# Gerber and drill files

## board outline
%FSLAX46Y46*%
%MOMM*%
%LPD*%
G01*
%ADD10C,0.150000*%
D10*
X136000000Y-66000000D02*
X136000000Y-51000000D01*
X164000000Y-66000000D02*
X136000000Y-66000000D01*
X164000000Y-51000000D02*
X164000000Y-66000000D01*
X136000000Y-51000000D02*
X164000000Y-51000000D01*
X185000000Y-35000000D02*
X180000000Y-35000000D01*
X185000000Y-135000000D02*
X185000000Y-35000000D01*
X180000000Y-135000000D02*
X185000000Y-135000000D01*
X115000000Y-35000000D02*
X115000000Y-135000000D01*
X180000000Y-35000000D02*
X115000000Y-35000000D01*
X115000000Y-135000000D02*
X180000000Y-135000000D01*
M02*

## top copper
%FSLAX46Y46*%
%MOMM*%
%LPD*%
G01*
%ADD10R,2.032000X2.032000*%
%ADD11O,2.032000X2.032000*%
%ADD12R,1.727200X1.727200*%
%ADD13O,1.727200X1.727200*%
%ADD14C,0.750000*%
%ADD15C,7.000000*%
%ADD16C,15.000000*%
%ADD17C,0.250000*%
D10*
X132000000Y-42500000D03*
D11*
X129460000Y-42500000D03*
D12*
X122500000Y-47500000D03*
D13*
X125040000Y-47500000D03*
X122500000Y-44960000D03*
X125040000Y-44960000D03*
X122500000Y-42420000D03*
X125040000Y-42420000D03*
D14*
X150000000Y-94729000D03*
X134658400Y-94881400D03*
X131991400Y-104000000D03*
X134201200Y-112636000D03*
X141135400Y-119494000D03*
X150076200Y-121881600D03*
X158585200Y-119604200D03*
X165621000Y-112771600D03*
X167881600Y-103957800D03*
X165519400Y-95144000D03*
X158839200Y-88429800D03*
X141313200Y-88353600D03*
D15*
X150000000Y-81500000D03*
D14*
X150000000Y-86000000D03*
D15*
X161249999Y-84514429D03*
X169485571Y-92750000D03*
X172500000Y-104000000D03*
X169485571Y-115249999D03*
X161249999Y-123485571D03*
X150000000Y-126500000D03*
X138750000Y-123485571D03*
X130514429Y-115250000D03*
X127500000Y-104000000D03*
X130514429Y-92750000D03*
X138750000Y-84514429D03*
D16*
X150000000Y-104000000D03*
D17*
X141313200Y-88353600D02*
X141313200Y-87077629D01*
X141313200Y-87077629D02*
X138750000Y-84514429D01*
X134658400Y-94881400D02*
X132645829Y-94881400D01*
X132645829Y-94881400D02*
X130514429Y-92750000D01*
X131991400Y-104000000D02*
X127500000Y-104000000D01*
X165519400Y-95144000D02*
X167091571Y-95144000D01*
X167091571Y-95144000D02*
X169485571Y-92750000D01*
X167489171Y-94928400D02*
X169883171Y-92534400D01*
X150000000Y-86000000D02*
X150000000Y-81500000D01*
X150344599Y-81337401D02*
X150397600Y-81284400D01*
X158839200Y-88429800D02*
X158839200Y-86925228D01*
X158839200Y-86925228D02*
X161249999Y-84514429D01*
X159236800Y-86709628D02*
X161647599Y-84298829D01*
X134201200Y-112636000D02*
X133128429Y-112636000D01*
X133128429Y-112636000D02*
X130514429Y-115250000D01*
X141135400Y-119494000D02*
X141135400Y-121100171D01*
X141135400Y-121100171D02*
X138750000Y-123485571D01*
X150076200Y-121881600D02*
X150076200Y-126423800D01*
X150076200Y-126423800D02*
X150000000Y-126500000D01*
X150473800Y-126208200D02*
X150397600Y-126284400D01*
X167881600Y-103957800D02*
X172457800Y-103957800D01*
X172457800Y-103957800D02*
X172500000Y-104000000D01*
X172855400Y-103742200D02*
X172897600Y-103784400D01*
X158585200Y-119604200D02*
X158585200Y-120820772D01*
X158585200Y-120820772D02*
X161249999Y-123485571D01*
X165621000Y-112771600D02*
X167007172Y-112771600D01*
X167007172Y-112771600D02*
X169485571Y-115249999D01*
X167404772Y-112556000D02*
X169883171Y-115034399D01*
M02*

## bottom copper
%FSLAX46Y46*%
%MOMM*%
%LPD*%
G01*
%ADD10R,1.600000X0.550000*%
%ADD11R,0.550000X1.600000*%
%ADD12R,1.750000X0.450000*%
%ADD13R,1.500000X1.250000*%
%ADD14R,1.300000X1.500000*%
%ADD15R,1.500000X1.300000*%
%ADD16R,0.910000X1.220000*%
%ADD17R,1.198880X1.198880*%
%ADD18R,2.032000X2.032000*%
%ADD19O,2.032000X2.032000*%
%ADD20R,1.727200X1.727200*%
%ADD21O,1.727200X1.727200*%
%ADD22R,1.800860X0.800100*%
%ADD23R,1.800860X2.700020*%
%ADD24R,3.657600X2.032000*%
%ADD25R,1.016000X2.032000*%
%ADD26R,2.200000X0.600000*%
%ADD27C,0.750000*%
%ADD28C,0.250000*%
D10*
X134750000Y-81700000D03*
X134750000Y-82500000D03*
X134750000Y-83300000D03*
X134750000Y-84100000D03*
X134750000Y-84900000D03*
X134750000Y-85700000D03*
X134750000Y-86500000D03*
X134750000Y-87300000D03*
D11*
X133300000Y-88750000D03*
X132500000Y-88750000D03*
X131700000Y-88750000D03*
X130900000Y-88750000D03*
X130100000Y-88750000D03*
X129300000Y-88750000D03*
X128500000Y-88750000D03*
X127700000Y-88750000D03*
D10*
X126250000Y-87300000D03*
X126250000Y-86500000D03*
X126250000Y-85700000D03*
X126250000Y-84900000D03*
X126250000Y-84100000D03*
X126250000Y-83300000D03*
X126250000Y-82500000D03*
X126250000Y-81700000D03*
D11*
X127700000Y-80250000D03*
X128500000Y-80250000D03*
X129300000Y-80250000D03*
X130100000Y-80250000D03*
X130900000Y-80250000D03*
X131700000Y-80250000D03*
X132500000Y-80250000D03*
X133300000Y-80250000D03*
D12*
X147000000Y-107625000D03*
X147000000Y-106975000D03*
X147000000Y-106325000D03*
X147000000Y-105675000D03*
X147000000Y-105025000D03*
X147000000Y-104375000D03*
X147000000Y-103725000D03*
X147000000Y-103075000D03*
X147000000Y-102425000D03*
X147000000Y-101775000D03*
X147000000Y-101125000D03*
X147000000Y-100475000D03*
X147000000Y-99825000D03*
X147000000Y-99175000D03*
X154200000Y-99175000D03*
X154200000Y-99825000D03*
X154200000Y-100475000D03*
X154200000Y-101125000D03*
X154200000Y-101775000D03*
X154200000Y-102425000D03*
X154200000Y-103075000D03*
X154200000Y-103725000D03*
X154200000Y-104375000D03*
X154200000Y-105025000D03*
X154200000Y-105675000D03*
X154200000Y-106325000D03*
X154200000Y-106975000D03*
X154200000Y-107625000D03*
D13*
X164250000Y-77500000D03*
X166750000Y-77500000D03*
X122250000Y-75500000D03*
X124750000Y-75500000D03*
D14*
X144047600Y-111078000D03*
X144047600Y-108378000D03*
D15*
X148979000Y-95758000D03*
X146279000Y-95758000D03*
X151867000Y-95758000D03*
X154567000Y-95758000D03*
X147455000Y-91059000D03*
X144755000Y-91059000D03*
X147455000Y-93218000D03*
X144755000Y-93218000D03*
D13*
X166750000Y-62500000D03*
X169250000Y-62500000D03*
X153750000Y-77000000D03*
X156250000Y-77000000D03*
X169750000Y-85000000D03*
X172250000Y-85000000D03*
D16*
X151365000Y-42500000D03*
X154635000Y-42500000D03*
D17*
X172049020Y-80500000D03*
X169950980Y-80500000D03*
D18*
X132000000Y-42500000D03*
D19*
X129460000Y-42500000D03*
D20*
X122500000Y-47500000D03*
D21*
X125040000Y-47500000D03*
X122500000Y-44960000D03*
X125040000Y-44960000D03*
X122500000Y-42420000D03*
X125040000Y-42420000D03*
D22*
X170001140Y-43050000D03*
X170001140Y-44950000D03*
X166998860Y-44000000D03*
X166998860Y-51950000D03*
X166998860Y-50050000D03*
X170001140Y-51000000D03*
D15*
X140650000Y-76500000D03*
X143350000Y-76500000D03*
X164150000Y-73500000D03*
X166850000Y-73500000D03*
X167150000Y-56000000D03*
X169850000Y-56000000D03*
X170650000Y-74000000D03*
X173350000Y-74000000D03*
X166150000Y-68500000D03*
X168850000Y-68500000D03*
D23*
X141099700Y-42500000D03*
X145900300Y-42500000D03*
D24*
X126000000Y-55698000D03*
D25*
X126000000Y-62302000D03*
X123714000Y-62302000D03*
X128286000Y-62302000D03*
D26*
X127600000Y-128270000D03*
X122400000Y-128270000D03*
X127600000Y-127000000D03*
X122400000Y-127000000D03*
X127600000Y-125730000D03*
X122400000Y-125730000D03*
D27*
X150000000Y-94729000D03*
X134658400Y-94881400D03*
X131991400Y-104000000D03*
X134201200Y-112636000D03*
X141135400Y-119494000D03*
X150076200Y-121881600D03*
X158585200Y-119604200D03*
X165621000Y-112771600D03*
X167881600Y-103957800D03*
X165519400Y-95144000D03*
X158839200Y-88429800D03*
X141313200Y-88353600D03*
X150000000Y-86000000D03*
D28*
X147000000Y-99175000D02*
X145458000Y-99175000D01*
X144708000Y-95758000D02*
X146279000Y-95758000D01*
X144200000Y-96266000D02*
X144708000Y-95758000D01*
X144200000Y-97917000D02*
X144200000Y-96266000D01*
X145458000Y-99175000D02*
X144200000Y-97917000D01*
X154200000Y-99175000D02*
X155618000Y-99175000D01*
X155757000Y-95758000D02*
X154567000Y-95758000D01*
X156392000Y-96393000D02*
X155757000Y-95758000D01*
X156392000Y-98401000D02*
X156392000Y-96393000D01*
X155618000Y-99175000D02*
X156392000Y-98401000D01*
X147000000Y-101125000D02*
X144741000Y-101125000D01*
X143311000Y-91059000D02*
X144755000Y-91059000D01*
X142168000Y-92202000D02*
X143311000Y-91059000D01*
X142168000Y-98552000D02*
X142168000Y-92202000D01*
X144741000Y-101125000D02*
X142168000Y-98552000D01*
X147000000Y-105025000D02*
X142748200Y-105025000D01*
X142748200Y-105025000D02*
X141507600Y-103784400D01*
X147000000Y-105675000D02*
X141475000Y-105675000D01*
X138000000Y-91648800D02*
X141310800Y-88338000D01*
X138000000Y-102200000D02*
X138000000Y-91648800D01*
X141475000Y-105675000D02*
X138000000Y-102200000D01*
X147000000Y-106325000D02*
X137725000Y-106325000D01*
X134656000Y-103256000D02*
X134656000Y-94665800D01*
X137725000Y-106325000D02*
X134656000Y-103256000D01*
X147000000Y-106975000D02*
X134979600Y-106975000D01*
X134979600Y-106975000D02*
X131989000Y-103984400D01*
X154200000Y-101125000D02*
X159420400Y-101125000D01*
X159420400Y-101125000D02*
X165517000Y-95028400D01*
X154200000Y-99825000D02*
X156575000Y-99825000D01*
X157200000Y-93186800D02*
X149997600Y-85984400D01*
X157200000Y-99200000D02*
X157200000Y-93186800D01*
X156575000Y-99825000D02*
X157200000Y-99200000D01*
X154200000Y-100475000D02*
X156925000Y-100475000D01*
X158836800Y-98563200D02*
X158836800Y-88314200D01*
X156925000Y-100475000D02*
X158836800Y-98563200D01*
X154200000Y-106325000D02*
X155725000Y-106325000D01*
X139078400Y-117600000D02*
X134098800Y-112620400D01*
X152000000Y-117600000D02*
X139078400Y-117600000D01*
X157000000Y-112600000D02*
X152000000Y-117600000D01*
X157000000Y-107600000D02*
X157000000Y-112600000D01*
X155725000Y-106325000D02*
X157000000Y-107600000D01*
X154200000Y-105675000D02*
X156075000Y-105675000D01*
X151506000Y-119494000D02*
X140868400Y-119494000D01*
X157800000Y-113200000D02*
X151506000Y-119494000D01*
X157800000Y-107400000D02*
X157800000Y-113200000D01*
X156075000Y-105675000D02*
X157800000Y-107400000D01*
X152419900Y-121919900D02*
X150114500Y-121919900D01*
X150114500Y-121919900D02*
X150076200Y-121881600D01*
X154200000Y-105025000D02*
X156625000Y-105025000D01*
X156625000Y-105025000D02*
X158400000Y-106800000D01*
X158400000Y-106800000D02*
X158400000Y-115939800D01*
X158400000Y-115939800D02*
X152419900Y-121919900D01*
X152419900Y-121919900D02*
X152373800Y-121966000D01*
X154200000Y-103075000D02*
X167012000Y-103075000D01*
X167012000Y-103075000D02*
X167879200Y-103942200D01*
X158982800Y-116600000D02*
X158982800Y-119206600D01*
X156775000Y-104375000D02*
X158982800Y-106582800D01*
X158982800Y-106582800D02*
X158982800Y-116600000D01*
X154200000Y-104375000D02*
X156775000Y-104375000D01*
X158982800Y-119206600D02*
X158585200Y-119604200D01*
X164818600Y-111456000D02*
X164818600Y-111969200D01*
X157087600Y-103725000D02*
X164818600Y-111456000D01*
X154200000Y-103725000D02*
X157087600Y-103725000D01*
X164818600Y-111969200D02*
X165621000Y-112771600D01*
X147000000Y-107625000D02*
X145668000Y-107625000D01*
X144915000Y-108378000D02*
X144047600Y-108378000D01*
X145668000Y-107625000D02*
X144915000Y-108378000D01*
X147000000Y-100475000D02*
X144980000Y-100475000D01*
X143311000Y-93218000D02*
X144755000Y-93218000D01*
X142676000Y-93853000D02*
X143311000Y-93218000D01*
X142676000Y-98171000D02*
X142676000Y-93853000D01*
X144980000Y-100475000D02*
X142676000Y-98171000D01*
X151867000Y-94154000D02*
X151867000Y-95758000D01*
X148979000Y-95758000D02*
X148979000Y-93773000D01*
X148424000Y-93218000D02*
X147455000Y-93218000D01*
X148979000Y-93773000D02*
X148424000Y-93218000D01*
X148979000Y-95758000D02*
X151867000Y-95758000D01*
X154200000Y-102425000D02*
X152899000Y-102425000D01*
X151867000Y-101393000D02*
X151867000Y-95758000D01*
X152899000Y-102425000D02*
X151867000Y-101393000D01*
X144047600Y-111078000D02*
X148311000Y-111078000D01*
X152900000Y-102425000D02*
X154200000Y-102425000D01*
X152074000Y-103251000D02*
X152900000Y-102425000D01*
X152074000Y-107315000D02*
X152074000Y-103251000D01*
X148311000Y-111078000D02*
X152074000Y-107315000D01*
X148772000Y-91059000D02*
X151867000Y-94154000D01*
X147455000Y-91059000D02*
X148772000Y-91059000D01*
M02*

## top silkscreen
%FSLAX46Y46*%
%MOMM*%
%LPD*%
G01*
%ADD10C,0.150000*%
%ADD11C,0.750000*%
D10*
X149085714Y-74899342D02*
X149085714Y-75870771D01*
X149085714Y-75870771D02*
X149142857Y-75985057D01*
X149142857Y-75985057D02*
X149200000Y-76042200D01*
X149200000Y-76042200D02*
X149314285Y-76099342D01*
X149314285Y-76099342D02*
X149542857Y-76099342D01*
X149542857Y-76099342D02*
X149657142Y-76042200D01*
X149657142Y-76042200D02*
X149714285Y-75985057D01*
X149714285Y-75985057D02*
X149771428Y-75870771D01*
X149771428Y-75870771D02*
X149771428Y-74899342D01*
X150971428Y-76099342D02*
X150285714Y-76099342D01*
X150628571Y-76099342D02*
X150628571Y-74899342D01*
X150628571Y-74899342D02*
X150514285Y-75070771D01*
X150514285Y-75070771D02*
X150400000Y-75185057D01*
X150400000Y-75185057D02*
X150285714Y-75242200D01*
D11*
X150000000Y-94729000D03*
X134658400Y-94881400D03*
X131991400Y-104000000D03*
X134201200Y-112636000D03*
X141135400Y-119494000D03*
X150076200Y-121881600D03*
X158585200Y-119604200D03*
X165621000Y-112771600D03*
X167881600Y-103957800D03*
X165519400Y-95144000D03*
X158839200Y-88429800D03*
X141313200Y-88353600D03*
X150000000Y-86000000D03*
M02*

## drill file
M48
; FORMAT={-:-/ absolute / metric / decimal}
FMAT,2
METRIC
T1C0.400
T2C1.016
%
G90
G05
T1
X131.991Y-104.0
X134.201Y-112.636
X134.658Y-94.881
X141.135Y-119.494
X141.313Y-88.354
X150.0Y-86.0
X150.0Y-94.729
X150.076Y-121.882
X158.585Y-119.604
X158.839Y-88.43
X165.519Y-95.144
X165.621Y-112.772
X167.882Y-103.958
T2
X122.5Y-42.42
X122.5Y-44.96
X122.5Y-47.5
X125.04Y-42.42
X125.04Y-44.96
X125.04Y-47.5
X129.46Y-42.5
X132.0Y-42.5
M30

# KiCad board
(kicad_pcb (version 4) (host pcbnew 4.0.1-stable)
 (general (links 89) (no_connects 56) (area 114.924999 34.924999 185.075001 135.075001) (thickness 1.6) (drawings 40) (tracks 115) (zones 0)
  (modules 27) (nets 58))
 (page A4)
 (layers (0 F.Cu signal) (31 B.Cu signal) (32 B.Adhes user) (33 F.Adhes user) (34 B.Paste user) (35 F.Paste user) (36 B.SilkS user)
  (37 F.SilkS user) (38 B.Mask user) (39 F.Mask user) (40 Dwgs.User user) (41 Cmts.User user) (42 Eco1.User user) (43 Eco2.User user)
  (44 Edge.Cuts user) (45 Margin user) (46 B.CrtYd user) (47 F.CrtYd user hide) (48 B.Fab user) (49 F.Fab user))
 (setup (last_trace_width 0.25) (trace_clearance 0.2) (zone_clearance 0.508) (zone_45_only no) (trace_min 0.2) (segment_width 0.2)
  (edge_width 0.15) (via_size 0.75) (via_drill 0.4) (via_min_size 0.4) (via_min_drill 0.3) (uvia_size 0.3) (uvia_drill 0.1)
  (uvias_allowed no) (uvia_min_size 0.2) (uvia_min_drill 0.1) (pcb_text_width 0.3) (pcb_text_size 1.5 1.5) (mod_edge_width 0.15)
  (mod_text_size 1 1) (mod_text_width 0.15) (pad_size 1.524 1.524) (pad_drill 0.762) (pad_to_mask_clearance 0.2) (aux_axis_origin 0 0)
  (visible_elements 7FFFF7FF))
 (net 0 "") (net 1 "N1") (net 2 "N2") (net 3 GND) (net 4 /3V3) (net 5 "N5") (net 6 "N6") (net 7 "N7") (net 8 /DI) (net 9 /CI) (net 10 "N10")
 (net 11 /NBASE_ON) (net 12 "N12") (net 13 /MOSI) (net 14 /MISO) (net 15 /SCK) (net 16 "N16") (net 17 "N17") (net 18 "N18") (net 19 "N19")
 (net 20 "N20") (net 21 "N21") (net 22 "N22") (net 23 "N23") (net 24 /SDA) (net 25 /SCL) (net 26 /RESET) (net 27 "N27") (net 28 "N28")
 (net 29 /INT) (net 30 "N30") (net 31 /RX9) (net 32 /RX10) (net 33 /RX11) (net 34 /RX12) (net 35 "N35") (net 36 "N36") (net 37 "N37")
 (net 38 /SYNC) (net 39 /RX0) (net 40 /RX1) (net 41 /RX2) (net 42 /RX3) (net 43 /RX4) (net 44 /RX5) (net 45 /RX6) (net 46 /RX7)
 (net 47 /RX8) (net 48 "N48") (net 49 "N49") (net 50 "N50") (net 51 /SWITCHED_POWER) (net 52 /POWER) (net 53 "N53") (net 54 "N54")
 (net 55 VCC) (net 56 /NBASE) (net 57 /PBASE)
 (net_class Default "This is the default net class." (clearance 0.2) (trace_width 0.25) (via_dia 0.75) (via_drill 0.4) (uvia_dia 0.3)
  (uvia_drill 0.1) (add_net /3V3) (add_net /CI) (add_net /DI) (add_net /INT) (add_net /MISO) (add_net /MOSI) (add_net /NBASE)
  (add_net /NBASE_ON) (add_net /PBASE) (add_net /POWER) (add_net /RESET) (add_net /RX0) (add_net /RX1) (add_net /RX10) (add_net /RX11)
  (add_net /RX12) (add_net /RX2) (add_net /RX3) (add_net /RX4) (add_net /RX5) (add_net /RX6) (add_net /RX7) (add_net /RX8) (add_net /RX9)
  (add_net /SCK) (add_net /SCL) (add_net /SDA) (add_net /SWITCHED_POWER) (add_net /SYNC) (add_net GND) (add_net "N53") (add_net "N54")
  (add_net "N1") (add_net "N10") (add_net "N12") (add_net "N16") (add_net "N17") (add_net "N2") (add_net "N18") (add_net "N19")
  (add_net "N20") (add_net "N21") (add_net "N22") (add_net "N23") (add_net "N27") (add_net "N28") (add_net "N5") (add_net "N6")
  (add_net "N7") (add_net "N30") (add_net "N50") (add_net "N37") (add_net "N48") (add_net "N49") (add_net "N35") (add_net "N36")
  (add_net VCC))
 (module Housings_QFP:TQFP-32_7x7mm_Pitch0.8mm (layer B.Cu) (at 130.5 84.5 180)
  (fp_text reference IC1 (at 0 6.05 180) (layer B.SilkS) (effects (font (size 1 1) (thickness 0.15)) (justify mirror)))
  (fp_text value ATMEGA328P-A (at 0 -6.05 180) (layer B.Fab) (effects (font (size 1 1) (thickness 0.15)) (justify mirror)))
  (pad 1 smd rect (at -4.25 2.8 180) (size 1.6 0.55) (layers B.Cu B.Paste B.Mask) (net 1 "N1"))
  (pad 2 smd rect (at -4.25 2 180) (size 1.6 0.55) (layers B.Cu B.Paste B.Mask) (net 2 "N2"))
  (pad 3 smd rect (at -4.25 1.2 180) (size 1.6 0.55) (layers B.Cu B.Paste B.Mask) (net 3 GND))
  (pad 4 smd rect (at -4.25 0.4 180) (size 1.6 0.55) (layers B.Cu B.Paste B.Mask) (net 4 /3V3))
  (pad 5 smd rect (at -4.25 -0.4 180) (size 1.6 0.55) (layers B.Cu B.Paste B.Mask) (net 3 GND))
  (pad 6 smd rect (at -4.25 -1.2 180) (size 1.6 0.55) (layers B.Cu B.Paste B.Mask) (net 4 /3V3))
  (pad 7 smd rect (at -4.25 -2 180) (size 1.6 0.55) (layers B.Cu B.Paste B.Mask) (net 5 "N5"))
  (pad 8 smd rect (at -4.25 -2.8 180) (size 1.6 0.55) (layers B.Cu B.Paste B.Mask) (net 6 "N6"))
  (pad 9 smd rect (at -2.8 -4.25 90) (size 1.6 0.55) (layers B.Cu B.Paste B.Mask) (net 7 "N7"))
  (pad 10 smd rect (at -2 -4.25 90) (size 1.6 0.55) (layers B.Cu B.Paste B.Mask) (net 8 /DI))
  (pad 11 smd rect (at -1.2 -4.25 90) (size 1.6 0.55) (layers B.Cu B.Paste B.Mask) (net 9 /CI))
  (pad 12 smd rect (at -0.4 -4.25 90) (size 1.6 0.55) (layers B.Cu B.Paste B.Mask) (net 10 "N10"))
  (pad 13 smd rect (at 0.4 -4.25 90) (size 1.6 0.55) (layers B.Cu B.Paste B.Mask) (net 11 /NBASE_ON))
  (pad 14 smd rect (at 1.2 -4.25 90) (size 1.6 0.55) (layers B.Cu B.Paste B.Mask) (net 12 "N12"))
  (pad 15 smd rect (at 2 -4.25 90) (size 1.6 0.55) (layers B.Cu B.Paste B.Mask) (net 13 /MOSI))
  (pad 16 smd rect (at 2.8 -4.25 90) (size 1.6 0.55) (layers B.Cu B.Paste B.Mask) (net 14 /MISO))
  (pad 17 smd rect (at 4.25 -2.8 180) (size 1.6 0.55) (layers B.Cu B.Paste B.Mask) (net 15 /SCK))
  (pad 18 smd rect (at 4.25 -2 180) (size 1.6 0.55) (layers B.Cu B.Paste B.Mask) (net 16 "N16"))
  (pad 19 smd rect (at 4.25 -1.2 180) (size 1.6 0.55) (layers B.Cu B.Paste B.Mask) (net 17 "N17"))
  (pad 20 smd rect (at 4.25 -0.4 180) (size 1.6 0.55) (layers B.Cu B.Paste B.Mask) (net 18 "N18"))
  (pad 21 smd rect (at 4.25 0.4 180) (size 1.6 0.55) (layers B.Cu B.Paste B.Mask) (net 3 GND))
  (pad 22 smd rect (at 4.25 1.2 180) (size 1.6 0.55) (layers B.Cu B.Paste B.Mask) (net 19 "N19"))
  (pad 23 smd rect (at 4.25 2 180) (size 1.6 0.55) (layers B.Cu B.Paste B.Mask) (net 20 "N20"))
  (pad 24 smd rect (at 4.25 2.8 180) (size 1.6 0.55) (layers B.Cu B.Paste B.Mask) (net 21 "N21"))
  (pad 25 smd rect (at 2.8 4.25 90) (size 1.6 0.55) (layers B.Cu B.Paste B.Mask) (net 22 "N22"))
  (pad 26 smd rect (at 2 4.25 90) (size 1.6 0.55) (layers B.Cu B.Paste B.Mask) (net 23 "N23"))
  (pad 27 smd rect (at 1.2 4.25 90) (size 1.6 0.55) (layers B.Cu B.Paste B.Mask) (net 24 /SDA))
  (pad 28 smd rect (at 0.4 4.25 90) (size 1.6 0.55) (layers B.Cu B.Paste B.Mask) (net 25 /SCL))
  (pad 29 smd rect (at -0.4 4.25 90) (size 1.6 0.55) (layers B.Cu B.Paste B.Mask) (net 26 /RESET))
  (pad 30 smd rect (at -1.2 4.25 90) (size 1.6 0.55) (layers B.Cu B.Paste B.Mask) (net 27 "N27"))
  (pad 31 smd rect (at -2 4.25 90) (size 1.6 0.55) (layers B.Cu B.Paste B.Mask) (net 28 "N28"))
  (pad 32 smd rect (at -2.8 4.25 90) (size 1.6 0.55) (layers B.Cu B.Paste B.Mask) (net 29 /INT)))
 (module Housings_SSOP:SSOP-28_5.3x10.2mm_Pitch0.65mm (layer B.Cu) (at 150.6 103.4)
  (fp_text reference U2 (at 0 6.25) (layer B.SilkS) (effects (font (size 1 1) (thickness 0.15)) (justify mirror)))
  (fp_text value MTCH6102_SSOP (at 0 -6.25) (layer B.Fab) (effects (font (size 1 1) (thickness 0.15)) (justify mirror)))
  (pad 1 smd rect (at -3.6 4.225) (size 1.75 0.45) (layers B.Cu B.Paste B.Mask) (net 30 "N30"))
  (pad 2 smd rect (at -3.6 3.575) (size 1.75 0.45) (layers B.Cu B.Paste B.Mask) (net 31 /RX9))
  (pad 3 smd rect (at -3.6 2.925) (size 1.75 0.45) (layers B.Cu B.Paste B.Mask) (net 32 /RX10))
  (pad 4 smd rect (at -3.6 2.275) (size 1.75 0.45) (layers B.Cu B.Paste B.Mask) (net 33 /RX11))
  (pad 5 smd rect (at -3.6 1.625) (size 1.75 0.45) (layers B.Cu B.Paste B.Mask) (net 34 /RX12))
  (pad 6 smd rect (at -3.6 0.975) (size 1.75 0.45) (layers B.Cu B.Paste B.Mask) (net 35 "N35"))
  (pad 7 smd rect (at -3.6 0.325) (size 1.75 0.45) (layers B.Cu B.Paste B.Mask) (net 3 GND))
  (pad 8 smd rect (at -3.6 -0.325) (size 1.75 0.45) (layers B.Cu B.Paste B.Mask) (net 3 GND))
  (pad 9 smd rect (at -3.6 -0.975) (size 1.75 0.45) (layers B.Cu B.Paste B.Mask) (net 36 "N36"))
  (pad 10 smd rect (at -3.6 -1.625) (size 1.75 0.45) (layers B.Cu B.Paste B.Mask) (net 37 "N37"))
  (pad 11 smd rect (at -3.6 -2.275) (size 1.75 0.45) (layers B.Cu B.Paste B.Mask) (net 29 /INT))
  (pad 12 smd rect (at -3.6 -2.925) (size 1.75 0.45) (layers B.Cu B.Paste B.Mask) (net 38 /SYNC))
  (pad 13 smd rect (at -3.6 -3.575) (size 1.75 0.45) (layers B.Cu B.Paste B.Mask) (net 3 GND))
  (pad 14 smd rect (at -3.6 -4.225) (size 1.75 0.45) (layers B.Cu B.Paste B.Mask) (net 24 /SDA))
  (pad 15 smd rect (at 3.6 -4.225) (size 1.75 0.45) (layers B.Cu B.Paste B.Mask) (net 25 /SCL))
  (pad 16 smd rect (at 3.6 -3.575) (size 1.75 0.45) (layers B.Cu B.Paste B.Mask) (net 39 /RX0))
  (pad 17 smd rect (at 3.6 -2.925) (size 1.75 0.45) (layers B.Cu B.Paste B.Mask) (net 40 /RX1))
  (pad 18 smd rect (at 3.6 -2.275) (size 1.75 0.45) (layers B.Cu B.Paste B.Mask) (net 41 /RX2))
  (pad 19 smd rect (at 3.6 -1.625) (size 1.75 0.45) (layers B.Cu B.Paste B.Mask) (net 3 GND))
  (pad 20 smd rect (at 3.6 -0.975) (size 1.75 0.45) (layers B.Cu B.Paste B.Mask) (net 4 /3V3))
  (pad 21 smd rect (at 3.6 -0.325) (size 1.75 0.45) (layers B.Cu B.Paste B.Mask) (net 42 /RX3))
  (pad 22 smd rect (at 3.6 0.325) (size 1.75 0.45) (layers B.Cu B.Paste B.Mask) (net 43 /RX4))
  (pad 23 smd rect (at 3.6 0.975) (size 1.75 0.45) (layers B.Cu B.Paste B.Mask) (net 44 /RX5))
  (pad 24 smd rect (at 3.6 1.625) (size 1.75 0.45) (layers B.Cu B.Paste B.Mask) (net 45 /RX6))
  (pad 25 smd rect (at 3.6 2.275) (size 1.75 0.45) (layers B.Cu B.Paste B.Mask) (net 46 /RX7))
  (pad 26 smd rect (at 3.6 2.925) (size 1.75 0.45) (layers B.Cu B.Paste B.Mask) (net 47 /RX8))
  (pad 27 smd rect (at 3.6 3.575) (size 1.75 0.45) (layers B.Cu B.Paste B.Mask) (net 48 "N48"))
  (pad 28 smd rect (at 3.6 4.225) (size 1.75 0.45) (layers B.Cu B.Paste B.Mask) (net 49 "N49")))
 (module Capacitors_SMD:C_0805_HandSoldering (layer B.Cu) (at 165.5 77.5)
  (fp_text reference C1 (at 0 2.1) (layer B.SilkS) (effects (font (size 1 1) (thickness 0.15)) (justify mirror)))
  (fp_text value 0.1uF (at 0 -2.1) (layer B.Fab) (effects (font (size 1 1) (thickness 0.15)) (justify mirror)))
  (pad 1 smd rect (at -1.25 0) (size 1.5 1.25) (layers B.Cu B.Paste B.Mask) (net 4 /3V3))
  (pad 2 smd rect (at 1.25 0) (size 1.5 1.25) (layers B.Cu B.Paste B.Mask) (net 3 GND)))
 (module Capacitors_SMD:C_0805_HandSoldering (layer B.Cu) (at 123.5 75.5)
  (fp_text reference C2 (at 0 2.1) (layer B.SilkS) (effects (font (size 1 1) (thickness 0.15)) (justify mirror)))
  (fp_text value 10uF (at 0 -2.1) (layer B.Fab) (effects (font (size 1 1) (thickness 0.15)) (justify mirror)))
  (pad 1 smd rect (at -1.25 0) (size 1.5 1.25) (layers B.Cu B.Paste B.Mask) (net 4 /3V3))
  (pad 2 smd rect (at 1.25 0) (size 1.5 1.25) (layers B.Cu B.Paste B.Mask) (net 3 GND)))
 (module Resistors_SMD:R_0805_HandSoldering (layer B.Cu) (at 144.0476 109.728 90)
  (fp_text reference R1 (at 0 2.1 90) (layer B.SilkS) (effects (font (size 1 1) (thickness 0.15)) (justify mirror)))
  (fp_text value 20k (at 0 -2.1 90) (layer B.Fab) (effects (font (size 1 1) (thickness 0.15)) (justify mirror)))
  (pad 1 smd rect (at -1.35 0 90) (size 1.5 1.3) (layers B.Cu B.Paste B.Mask) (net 4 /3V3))
  (pad 2 smd rect (at 1.35 0 90) (size 1.5 1.3) (layers B.Cu B.Paste B.Mask) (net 30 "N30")))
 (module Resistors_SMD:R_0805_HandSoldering (layer B.Cu) (at 147.629 95.758 180)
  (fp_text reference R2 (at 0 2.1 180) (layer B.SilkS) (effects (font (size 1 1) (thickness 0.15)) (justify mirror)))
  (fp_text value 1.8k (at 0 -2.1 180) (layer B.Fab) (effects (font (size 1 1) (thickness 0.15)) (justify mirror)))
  (pad 1 smd rect (at -1.35 0 180) (size 1.5 1.3) (layers B.Cu B.Paste B.Mask) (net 4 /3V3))
  (pad 2 smd rect (at 1.35 0 180) (size 1.5 1.3) (layers B.Cu B.Paste B.Mask) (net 24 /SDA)))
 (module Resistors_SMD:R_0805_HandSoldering (layer B.Cu) (at 153.217 95.758)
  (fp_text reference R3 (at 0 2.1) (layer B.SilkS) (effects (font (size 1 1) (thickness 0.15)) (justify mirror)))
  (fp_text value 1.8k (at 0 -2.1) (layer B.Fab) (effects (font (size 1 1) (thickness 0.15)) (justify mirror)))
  (pad 1 smd rect (at -1.35 0) (size 1.5 1.3) (layers B.Cu B.Paste B.Mask) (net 4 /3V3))
  (pad 2 smd rect (at 1.35 0) (size 1.5 1.3) (layers B.Cu B.Paste B.Mask) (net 25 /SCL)))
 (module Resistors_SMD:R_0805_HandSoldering (layer B.Cu) (at 146.105 91.059 180)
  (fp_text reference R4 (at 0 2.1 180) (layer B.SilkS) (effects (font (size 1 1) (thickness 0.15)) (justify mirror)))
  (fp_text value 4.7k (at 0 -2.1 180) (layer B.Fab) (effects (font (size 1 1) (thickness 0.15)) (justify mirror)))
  (pad 1 smd rect (at -1.35 0 180) (size 1.5 1.3) (layers B.Cu B.Paste B.Mask) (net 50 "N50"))
  (pad 2 smd rect (at 1.35 0 180) (size 1.5 1.3) (layers B.Cu B.Paste B.Mask) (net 29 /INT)))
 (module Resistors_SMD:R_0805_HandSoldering (layer B.Cu) (at 146.105 93.218 180)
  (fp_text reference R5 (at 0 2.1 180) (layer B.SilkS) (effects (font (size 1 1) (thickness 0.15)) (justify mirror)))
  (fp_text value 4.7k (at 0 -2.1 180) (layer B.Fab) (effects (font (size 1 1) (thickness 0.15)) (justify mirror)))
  (pad 1 smd rect (at -1.35 0 180) (size 1.5 1.3) (layers B.Cu B.Paste B.Mask) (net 4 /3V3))
  (pad 2 smd rect (at 1.35 0 180) (size 1.5 1.3) (layers B.Cu B.Paste B.Mask) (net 38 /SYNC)))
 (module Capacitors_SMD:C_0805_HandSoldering (layer B.Cu) (at 168 62.5)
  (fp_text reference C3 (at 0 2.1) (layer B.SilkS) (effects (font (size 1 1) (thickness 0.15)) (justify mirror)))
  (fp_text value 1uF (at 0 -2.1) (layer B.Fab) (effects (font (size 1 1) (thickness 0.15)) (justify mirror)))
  (pad 1 smd rect (at -1.25 0) (size 1.5 1.25) (layers B.Cu B.Paste B.Mask) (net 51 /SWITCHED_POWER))
  (pad 2 smd rect (at 1.25 0) (size 1.5 1.25) (layers B.Cu B.Paste B.Mask) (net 3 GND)))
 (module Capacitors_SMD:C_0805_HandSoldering (layer B.Cu) (at 155 77)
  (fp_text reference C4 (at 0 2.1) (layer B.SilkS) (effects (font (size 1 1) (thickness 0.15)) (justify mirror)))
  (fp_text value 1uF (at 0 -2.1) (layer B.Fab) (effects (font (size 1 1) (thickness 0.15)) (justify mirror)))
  (pad 1 smd rect (at -1.25 0) (size 1.5 1.25) (layers B.Cu B.Paste B.Mask) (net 4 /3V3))
  (pad 2 smd rect (at 1.25 0) (size 1.5 1.25) (layers B.Cu B.Paste B.Mask) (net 3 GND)))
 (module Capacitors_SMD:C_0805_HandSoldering (layer B.Cu) (at 171 85)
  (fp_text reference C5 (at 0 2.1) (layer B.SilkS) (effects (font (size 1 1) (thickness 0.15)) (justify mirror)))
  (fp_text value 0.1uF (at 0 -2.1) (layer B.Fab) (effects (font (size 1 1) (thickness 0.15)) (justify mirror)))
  (pad 1 smd rect (at -1.25 0) (size 1.5 1.25) (layers B.Cu B.Paste B.Mask) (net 4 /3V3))
  (pad 2 smd rect (at 1.25 0) (size 1.5 1.25) (layers B.Cu B.Paste B.Mask) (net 3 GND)))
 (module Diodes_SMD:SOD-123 (layer B.Cu) (at 153 42.5)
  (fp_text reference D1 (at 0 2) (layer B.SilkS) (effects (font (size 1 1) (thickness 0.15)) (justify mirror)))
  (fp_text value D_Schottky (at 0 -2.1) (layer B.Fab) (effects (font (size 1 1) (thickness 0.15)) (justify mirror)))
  (pad 1 smd rect (at -1.635 0) (size 0.91 1.22) (layers B.Cu B.Paste B.Mask) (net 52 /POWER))
  (pad 2 smd rect (at 1.635 0) (size 0.91 1.22) (layers B.Cu B.Paste B.Mask) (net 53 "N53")))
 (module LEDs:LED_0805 (layer B.Cu) (at 171 80.5)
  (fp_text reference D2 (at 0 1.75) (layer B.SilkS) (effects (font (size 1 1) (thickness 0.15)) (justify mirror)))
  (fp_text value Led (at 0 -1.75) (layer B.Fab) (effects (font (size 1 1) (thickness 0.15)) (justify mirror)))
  (pad 2 smd rect (at 1.04902 0 180) (size 1.19888 1.19888) (layers B.Cu B.Paste B.Mask) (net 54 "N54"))
  (pad 1 smd rect (at -1.04902 0 180) (size 1.19888 1.19888) (layers B.Cu B.Paste B.Mask) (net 3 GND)))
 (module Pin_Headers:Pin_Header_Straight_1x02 (layer B.Cu) (at 132 42.5 90)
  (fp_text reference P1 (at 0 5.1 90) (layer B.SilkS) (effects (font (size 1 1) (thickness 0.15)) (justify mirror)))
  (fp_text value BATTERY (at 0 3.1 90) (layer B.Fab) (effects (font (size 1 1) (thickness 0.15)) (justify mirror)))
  (pad 1 thru_hole rect (at 0 0 90) (size 2.032 2.032) (drill 1.016) (layers *.Cu *.Mask B.SilkS) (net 3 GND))
  (pad 2 thru_hole oval (at 0 -2.54 90) (size 2.032 2.032) (drill 1.016) (layers *.Cu *.Mask B.SilkS) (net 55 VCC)))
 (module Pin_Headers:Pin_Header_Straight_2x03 (layer B.Cu) (at 122.5 47.5)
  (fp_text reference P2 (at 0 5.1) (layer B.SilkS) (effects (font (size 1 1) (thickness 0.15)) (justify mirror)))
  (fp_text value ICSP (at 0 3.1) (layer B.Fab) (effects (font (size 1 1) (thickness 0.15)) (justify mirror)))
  (pad 1 thru_hole rect (at 0 0) (size 1.7272 1.7272) (drill 1.016) (layers *.Cu *.Mask B.SilkS) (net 14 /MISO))
  (pad 2 thru_hole oval (at 2.54 0) (size 1.7272 1.7272) (drill 1.016) (layers *.Cu *.Mask B.SilkS) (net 51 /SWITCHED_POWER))
  (pad 3 thru_hole oval (at 0 -2.54) (size 1.7272 1.7272) (drill 1.016) (layers *.Cu *.Mask B.SilkS) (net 15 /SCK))
  (pad 4 thru_hole oval (at 2.54 -2.54) (size 1.7272 1.7272) (drill 1.016) (layers *.Cu *.Mask B.SilkS) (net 13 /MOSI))
  (pad 5 thru_hole oval (at 0 -5.08) (size 1.7272 1.7272) (drill 1.016) (layers *.Cu *.Mask B.SilkS) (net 26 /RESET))
  (pad 6 thru_hole oval (at 2.54 -5.08) (size 1.7272 1.7272) (drill 1.016) (layers *.Cu *.Mask B.SilkS) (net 3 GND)))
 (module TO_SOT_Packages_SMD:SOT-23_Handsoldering (layer B.Cu) (at 168.5 44 270)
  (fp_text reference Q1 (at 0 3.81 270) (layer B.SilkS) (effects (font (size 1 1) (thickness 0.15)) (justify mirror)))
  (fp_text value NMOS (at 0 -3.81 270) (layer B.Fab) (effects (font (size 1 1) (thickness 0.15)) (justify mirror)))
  (pad 1 smd rect (at -0.95 -1.50114 270) (size 0.8001 1.80086) (layers B.Cu B.Paste B.Mask) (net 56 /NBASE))
  (pad 2 smd rect (at 0.95 -1.50114 270) (size 0.8001 1.80086) (layers B.Cu B.Paste B.Mask) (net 3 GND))
  (pad 3 smd rect (at 0 1.50114 270) (size 0.8001 1.80086) (layers B.Cu B.Paste B.Mask) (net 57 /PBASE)))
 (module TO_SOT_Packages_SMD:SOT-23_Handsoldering (layer B.Cu) (at 168.5 51 90)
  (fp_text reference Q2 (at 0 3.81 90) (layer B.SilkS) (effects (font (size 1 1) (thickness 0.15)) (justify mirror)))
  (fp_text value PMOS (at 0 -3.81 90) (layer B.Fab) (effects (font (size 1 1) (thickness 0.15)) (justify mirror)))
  (pad 1 smd rect (at -0.95 -1.50114 90) (size 0.8001 1.80086) (layers B.Cu B.Paste B.Mask) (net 57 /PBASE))
  (pad 2 smd rect (at 0.95 -1.50114 90) (size 0.8001 1.80086) (layers B.Cu B.Paste B.Mask) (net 51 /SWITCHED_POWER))
  (pad 3 smd rect (at 0 1.50114 90) (size 0.8001 1.80086) (layers B.Cu B.Paste B.Mask) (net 52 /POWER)))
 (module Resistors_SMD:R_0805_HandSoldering (layer B.Cu) (at 142 76.5)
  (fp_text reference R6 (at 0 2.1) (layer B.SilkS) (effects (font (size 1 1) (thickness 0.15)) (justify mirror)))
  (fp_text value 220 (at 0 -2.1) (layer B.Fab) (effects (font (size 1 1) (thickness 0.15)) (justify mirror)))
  (pad 1 smd rect (at -1.35 0) (size 1.5 1.3) (layers B.Cu B.Paste B.Mask) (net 56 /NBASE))
  (pad 2 smd rect (at 1.35 0) (size 1.5 1.3) (layers B.Cu B.Paste B.Mask) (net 11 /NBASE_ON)))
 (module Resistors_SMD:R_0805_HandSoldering (layer B.Cu) (at 165.5 73.5)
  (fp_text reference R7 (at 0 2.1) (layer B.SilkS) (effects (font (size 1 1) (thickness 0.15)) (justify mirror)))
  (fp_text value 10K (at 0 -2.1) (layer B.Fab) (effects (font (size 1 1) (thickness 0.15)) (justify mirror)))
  (pad 1 smd rect (at -1.35 0) (size 1.5 1.3) (layers B.Cu B.Paste B.Mask) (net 56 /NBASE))
  (pad 2 smd rect (at 1.35 0) (size 1.5 1.3) (layers B.Cu B.Paste B.Mask) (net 3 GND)))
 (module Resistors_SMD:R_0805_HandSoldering (layer B.Cu) (at 168.5 56)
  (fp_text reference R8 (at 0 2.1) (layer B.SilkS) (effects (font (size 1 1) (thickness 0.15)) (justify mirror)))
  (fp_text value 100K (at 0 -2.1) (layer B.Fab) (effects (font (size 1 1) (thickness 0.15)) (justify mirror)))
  (pad 1 smd rect (at -1.35 0) (size 1.5 1.3) (layers B.Cu B.Paste B.Mask) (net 52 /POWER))
  (pad 2 smd rect (at 1.35 0) (size 1.5 1.3) (layers B.Cu B.Paste B.Mask) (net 57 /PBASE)))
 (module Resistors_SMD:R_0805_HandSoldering (layer B.Cu) (at 172 74)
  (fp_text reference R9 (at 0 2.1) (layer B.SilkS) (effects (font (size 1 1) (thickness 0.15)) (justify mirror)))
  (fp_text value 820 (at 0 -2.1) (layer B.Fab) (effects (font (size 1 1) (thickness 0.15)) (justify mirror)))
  (pad 1 smd rect (at -1.35 0) (size 1.5 1.3) (layers B.Cu B.Paste B.Mask) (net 15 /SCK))
  (pad 2 smd rect (at 1.35 0) (size 1.5 1.3) (layers B.Cu B.Paste B.Mask) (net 54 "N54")))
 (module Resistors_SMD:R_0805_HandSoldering (layer B.Cu) (at 167.5 68.5)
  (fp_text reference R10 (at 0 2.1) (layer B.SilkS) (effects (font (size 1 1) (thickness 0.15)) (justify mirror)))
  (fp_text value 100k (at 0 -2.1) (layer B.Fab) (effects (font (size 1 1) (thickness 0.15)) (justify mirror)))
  (pad 1 smd rect (at -1.35 0) (size 1.5 1.3) (layers B.Cu B.Paste B.Mask) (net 26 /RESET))
  (pad 2 smd rect (at 1.35 0) (size 1.5 1.3) (layers B.Cu B.Paste B.Mask) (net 3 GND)))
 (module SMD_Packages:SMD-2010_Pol (layer B.Cu) (at 143.5 42.5)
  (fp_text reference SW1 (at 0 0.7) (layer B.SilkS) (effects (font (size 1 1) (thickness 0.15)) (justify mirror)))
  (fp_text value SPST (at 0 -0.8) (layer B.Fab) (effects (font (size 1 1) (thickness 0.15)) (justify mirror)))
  (pad 1 smd rect (at -2.4003 0) (size 1.80086 2.70002) (layers B.Cu B.Paste B.Mask) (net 53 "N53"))
  (pad 2 smd rect (at 2.4003 0) (size 1.80086 2.70002) (layers B.Cu B.Paste B.Mask) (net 55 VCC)))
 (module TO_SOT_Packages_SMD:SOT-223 (layer B.Cu) (at 126 59 180)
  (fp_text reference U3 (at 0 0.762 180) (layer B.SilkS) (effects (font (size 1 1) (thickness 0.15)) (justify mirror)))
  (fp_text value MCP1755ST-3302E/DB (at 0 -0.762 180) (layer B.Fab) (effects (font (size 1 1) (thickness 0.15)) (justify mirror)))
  (pad 4 smd rect (at 0 3.302 180) (size 3.6576 2.032) (layers B.Cu B.Paste B.Mask) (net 3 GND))
  (pad 2 smd rect (at 0 -3.302 180) (size 1.016 2.032) (layers B.Cu B.Paste B.Mask) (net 3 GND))
  (pad 3 smd rect (at 2.286 -3.302 180) (size 1.016 2.032) (layers B.Cu B.Paste B.Mask) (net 4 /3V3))
  (pad 1 smd rect (at -2.286 -3.302 180) (size 1.016 2.032) (layers B.Cu B.Paste B.Mask) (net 51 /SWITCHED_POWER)))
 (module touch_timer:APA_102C (layer B.Cu) (at 125 127 90)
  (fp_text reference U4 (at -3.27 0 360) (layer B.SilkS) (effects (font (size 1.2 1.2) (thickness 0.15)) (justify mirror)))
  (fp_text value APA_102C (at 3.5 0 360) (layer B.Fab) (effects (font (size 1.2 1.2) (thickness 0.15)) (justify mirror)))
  (pad 6 smd rect (at -1.27 2.6 90) (size 0.6 2.2) (layers B.Cu B.Paste B.Mask) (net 3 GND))
  (pad 1 smd rect (at -1.27 -2.6 90) (size 0.6 2.2) (layers B.Cu B.Paste B.Mask) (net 8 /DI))
  (pad 5 smd rect (at 0 2.6 90) (size 0.6 2.2) (layers B.Cu B.Paste B.Mask) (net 3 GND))
  (pad 2 smd rect (at 0 -2.6 90) (size 0.6 2.2) (layers B.Cu B.Paste B.Mask) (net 9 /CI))
  (pad 4 smd rect (at 1.27 2.6 90) (size 0.6 2.2) (layers B.Cu B.Paste B.Mask) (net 52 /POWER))
  (pad 3 smd rect (at 1.27 -2.6 90) (size 0.6 2.2) (layers B.Cu B.Paste B.Mask) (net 3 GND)))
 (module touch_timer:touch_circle (layer F.Cu) (at 150 104)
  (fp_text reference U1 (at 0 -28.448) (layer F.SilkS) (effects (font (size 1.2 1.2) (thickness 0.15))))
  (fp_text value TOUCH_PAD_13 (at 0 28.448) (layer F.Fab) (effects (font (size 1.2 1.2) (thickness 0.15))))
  (pad 13 thru_hole circle (at 0 -9.271) (size 0.75 0.75) (drill 0.4) (layers *.Cu *.Mask F.SilkS) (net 34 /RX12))
  (pad 11 thru_hole circle (at -15.3416 -9.1186) (size 0.75 0.75) (drill 0.4) (layers *.Cu *.Mask F.SilkS) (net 32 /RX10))
  (pad 10 thru_hole circle (at -18.0086 0) (size 0.75 0.75) (drill 0.4) (layers *.Cu *.Mask F.SilkS) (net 31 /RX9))
  (pad 9 thru_hole circle (at -15.7988 8.636) (size 0.75 0.75) (drill 0.4) (layers *.Cu *.Mask F.SilkS) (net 47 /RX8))
  (pad 8 thru_hole circle (at -8.8646 15.494) (size 0.75 0.75) (drill 0.4) (layers *.Cu *.Mask F.SilkS) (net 46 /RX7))
  (pad 7 thru_hole circle (at 0.0762 17.8816) (size 0.75 0.75) (drill 0.4) (layers *.Cu *.Mask F.SilkS) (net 45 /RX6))
  (pad 6 thru_hole circle (at 8.5852 15.6042) (size 0.75 0.75) (drill 0.4) (layers *.Cu *.Mask F.SilkS) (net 44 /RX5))
  (pad 5 thru_hole circle (at 15.621 8.7716) (size 0.75 0.75) (drill 0.4) (layers *.Cu *.Mask F.SilkS) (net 43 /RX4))
  (pad 4 thru_hole circle (at 17.8816 -0.0422) (size 0.75 0.75) (drill 0.4) (layers *.Cu *.Mask F.SilkS) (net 42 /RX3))
  (pad 3 thru_hole circle (at 15.5194 -8.856) (size 0.75 0.75) (drill 0.4) (layers *.Cu *.Mask F.SilkS) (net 41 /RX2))
  (pad 2 thru_hole circle (at 8.8392 -15.5702) (size 0.75 0.75) (drill 0.4) (layers *.Cu *.Mask F.SilkS) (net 40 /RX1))
  (pad 12 thru_hole circle (at -8.6868 -15.6464) (size 0.75 0.75) (drill 0.4) (layers *.Cu *.Mask F.SilkS) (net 33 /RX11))
  (pad 1 smd circle (at 0 -22.5) (size 7 7) (layers F.Cu) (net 39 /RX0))
  (pad 1 thru_hole circle (at 0 -18) (size 0.75 0.75) (drill 0.4) (layers *.Cu *.Mask F.SilkS) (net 39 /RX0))
  (pad 2 smd circle (at 11.249999 -19.485571) (size 7 7) (layers F.Cu) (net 40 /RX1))
  (pad 3 smd circle (at 19.485571 -11.25) (size 7 7) (layers F.Cu) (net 41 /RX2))
  (pad 4 smd circle (at 22.5 0) (size 7 7) (layers F.Cu) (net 42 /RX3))
  (pad 5 smd circle (at 19.485571 11.249999) (size 7 7) (layers F.Cu) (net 43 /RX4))
  (pad 6 smd circle (at 11.249999 19.485571) (size 7 7) (layers F.Cu) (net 44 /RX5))
  (pad 7 smd circle (at 0 22.5) (size 7 7) (layers F.Cu) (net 45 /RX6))
  (pad 8 smd circle (at -11.25 19.485571) (size 7 7) (layers F.Cu) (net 46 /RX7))
  (pad 9 smd circle (at -19.485571 11.25) (size 7 7) (layers F.Cu) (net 47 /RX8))
  (pad 10 smd circle (at -22.5 0) (size 7 7) (layers F.Cu) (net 31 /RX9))
  (pad 11 smd circle (at -19.485571 -11.25) (size 7 7) (layers F.Cu) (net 32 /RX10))
  (pad 12 smd circle (at -11.25 -19.485571) (size 7 7) (layers F.Cu) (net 33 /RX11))
  (pad 13 smd circle (at 0 0) (size 15 15) (layers F.Cu) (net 34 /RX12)))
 (gr_line (start 136 66) (end 136 51) (angle 90) (layer Edge.Cuts) (width 0.15))
 (gr_line (start 164 66) (end 136 66) (angle 90) (layer Edge.Cuts) (width 0.15))
 (gr_line (start 164 51) (end 164 66) (angle 90) (layer Edge.Cuts) (width 0.15))
 (gr_line (start 136 51) (end 164 51) (angle 90) (layer Edge.Cuts) (width 0.15))
 (gr_line (start 185 35) (end 180 35) (angle 90) (layer Edge.Cuts) (width 0.15))
 (gr_line (start 185 135) (end 185 35) (angle 90) (layer Edge.Cuts) (width 0.15))
 (gr_line (start 180 135) (end 185 135) (angle 90) (layer Edge.Cuts) (width 0.15))
 (gr_line (start 115 35) (end 115 135) (angle 90) (layer Edge.Cuts) (width 0.15))
 (gr_line (start 180 35) (end 115 35) (angle 90) (layer Edge.Cuts) (width 0.15))
 (gr_line (start 115 135) (end 180 135) (angle 90) (layer Edge.Cuts) (width 0.15))
 (segment (start 147 99.175) (end 145.458 99.175) (width 0.25) (layer B.Cu) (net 24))
 (segment (start 144.708 95.758) (end 146.279 95.758) (width 0.25) (layer B.Cu) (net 24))
 (segment (start 144.2 96.266) (end 144.708 95.758) (width 0.25) (layer B.Cu) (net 24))
 (segment (start 144.2 97.917) (end 144.2 96.266) (width 0.25) (layer B.Cu) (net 24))
 (segment (start 145.458 99.175) (end 144.2 97.917) (width 0.25) (layer B.Cu) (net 24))
 (segment (start 154.2 99.175) (end 155.618 99.175) (width 0.25) (layer B.Cu) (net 25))
 (segment (start 155.757 95.758) (end 154.567 95.758) (width 0.25) (layer B.Cu) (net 25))
 (segment (start 156.392 96.393) (end 155.757 95.758) (width 0.25) (layer B.Cu) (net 25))
 (segment (start 156.392 98.401) (end 156.392 96.393) (width 0.25) (layer B.Cu) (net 25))
 (segment (start 155.618 99.175) (end 156.392 98.401) (width 0.25) (layer B.Cu) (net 25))
 (segment (start 147 101.125) (end 144.741 101.125) (width 0.25) (layer B.Cu) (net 29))
 (segment (start 143.311 91.059) (end 144.755 91.059) (width 0.25) (layer B.Cu) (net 29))
 (segment (start 142.168 92.202) (end 143.311 91.059) (width 0.25) (layer B.Cu) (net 29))
 (segment (start 142.168 98.552) (end 142.168 92.202) (width 0.25) (layer B.Cu) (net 29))
 (segment (start 144.741 101.125) (end 142.168 98.552) (width 0.25) (layer B.Cu) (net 29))
 (segment (start 147 105.025) (end 142.7482 105.025) (width 0.25) (layer B.Cu) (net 34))
 (segment (start 142.7482 105.025) (end 141.5076 103.7844) (width 0.25) (layer B.Cu) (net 34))
 (segment (start 141.3132 88.3536) (end 141.3132 87.077629) (width 0.25) (layer F.Cu) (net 33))
 (segment (start 141.3132 87.077629) (end 138.75 84.514429) (width 0.25) (layer F.Cu) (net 33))
 (segment (start 147 105.675) (end 141.475 105.675) (width 0.25) (layer B.Cu) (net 33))
 (segment (start 138 91.6488) (end 141.3108 88.338) (width 0.25) (layer B.Cu) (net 33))
 (segment (start 138 102.2) (end 138 91.6488) (width 0.25) (layer B.Cu) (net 33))
 (segment (start 141.475 105.675) (end 138 102.2) (width 0.25) (layer B.Cu) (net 33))
 (segment (start 134.6584 94.8814) (end 132.645829 94.8814) (width 0.25) (layer F.Cu) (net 32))
 (segment (start 132.645829 94.8814) (end 130.514429 92.75) (width 0.25) (layer F.Cu) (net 32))
 (segment (start 147 106.325) (end 137.725 106.325) (width 0.25) (layer B.Cu) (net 32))
 (segment (start 134.656 103.256) (end 134.656 94.6658) (width 0.25) (layer B.Cu) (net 32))
 (segment (start 137.725 106.325) (end 134.656 103.256) (width 0.25) (layer B.Cu) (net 32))
 (segment (start 131.9914 104) (end 127.5 104) (width 0.25) (layer F.Cu) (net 31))
 (segment (start 147 106.975) (end 134.9796 106.975) (width 0.25) (layer B.Cu) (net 31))
 (segment (start 134.9796 106.975) (end 131.989 103.9844) (width 0.25) (layer B.Cu) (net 31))
 (segment (start 165.5194 95.144) (end 167.091571 95.144) (width 0.25) (layer F.Cu) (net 41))
 (segment (start 167.091571 95.144) (end 169.485571 92.75) (width 0.25) (layer F.Cu) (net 41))
 (segment (start 167.489171 94.9284) (end 169.883171 92.5344) (width 0.25) (layer F.Cu) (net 41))
 (segment (start 154.2 101.125) (end 159.4204 101.125) (width 0.25) (layer B.Cu) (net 41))
 (segment (start 159.4204 101.125) (end 165.517 95.0284) (width 0.25) (layer B.Cu) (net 41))
 (segment (start 150 86) (end 150 81.5) (width 0.25) (layer F.Cu) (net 39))
 (segment (start 150.344599 81.337401) (end 150.3976 81.2844) (width 0.25) (layer F.Cu) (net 39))
 (segment (start 154.2 99.825) (end 156.575 99.825) (width 0.25) (layer B.Cu) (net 39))
 (segment (start 157.2 93.1868) (end 149.9976 85.9844) (width 0.25) (layer B.Cu) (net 39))
 (segment (start 157.2 99.2) (end 157.2 93.1868) (width 0.25) (layer B.Cu) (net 39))
 (segment (start 156.575 99.825) (end 157.2 99.2) (width 0.25) (layer B.Cu) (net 39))
 (segment (start 158.8392 88.4298) (end 158.8392 86.925228) (width 0.25) (layer F.Cu) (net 40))
 (segment (start 158.8392 86.925228) (end 161.249999 84.514429) (width 0.25) (layer F.Cu) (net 40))
 (segment (start 159.2368 86.709628) (end 161.647599 84.298829) (width 0.25) (layer F.Cu) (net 40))
 (segment (start 154.2 100.475) (end 156.925 100.475) (width 0.25) (layer B.Cu) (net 40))
 (segment (start 158.8368 98.5632) (end 158.8368 88.3142) (width 0.25) (layer B.Cu) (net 40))
 (segment (start 156.925 100.475) (end 158.8368 98.5632) (width 0.25) (layer B.Cu) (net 40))
 (segment (start 134.2012 112.636) (end 133.128429 112.636) (width 0.25) (layer F.Cu) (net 47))
 (segment (start 133.128429 112.636) (end 130.514429 115.25) (width 0.25) (layer F.Cu) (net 47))
 (segment (start 154.2 106.325) (end 155.725 106.325) (width 0.25) (layer B.Cu) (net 47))
 (segment (start 139.0784 117.6) (end 134.0988 112.6204) (width 0.25) (layer B.Cu) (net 47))
 (segment (start 152 117.6) (end 139.0784 117.6) (width 0.25) (layer B.Cu) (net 47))
 (segment (start 157 112.6) (end 152 117.6) (width 0.25) (layer B.Cu) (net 47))
 (segment (start 157 107.6) (end 157 112.6) (width 0.25) (layer B.Cu) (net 47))
 (segment (start 155.725 106.325) (end 157 107.6) (width 0.25) (layer B.Cu) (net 47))
 (segment (start 141.1354 119.494) (end 141.1354 121.100171) (width 0.25) (layer F.Cu) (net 46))
 (segment (start 141.1354 121.100171) (end 138.75 123.485571) (width 0.25) (layer F.Cu) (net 46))
 (segment (start 154.2 105.675) (end 156.075 105.675) (width 0.25) (layer B.Cu) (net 46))
 (segment (start 151.506 119.494) (end 140.8684 119.494) (width 0.25) (layer B.Cu) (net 46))
 (segment (start 157.8 113.2) (end 151.506 119.494) (width 0.25) (layer B.Cu) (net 46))
 (segment (start 157.8 107.4) (end 157.8 113.2) (width 0.25) (layer B.Cu) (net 46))
 (segment (start 156.075 105.675) (end 157.8 107.4) (width 0.25) (layer B.Cu) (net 46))
 (segment (start 150.0762 121.8816) (end 150.0762 126.4238) (width 0.25) (layer F.Cu) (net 45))
 (segment (start 150.0762 126.4238) (end 150 126.5) (width 0.25) (layer F.Cu) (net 45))
 (segment (start 152.4199 121.9199) (end 150.1145 121.9199) (width 0.25) (layer B.Cu) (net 45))
 (segment (start 150.1145 121.9199) (end 150.0762 121.8816) (width 0.25) (layer B.Cu) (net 45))
 (segment (start 154.2 105.025) (end 156.625 105.025) (width 0.25) (layer B.Cu) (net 45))
 (segment (start 156.625 105.025) (end 158.4 106.8) (width 0.25) (layer B.Cu) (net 45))
 (segment (start 158.4 106.8) (end 158.4 115.9398) (width 0.25) (layer B.Cu) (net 45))
 (segment (start 158.4 115.9398) (end 152.4199 121.9199) (width 0.25) (layer B.Cu) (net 45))
 (segment (start 152.4199 121.9199) (end 152.3738 121.966) (width 0.25) (layer B.Cu) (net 45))
 (segment (start 150.4738 126.2082) (end 150.3976 126.2844) (width 0.25) (layer F.Cu) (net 45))
 (segment (start 167.8816 103.9578) (end 172.4578 103.9578) (width 0.25) (layer F.Cu) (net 42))
 (segment (start 172.4578 103.9578) (end 172.5 104) (width 0.25) (layer F.Cu) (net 42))
 (segment (start 172.8554 103.7422) (end 172.8976 103.7844) (width 0.25) (layer F.Cu) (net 42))
 (segment (start 154.2 103.075) (end 167.012 103.075) (width 0.25) (layer B.Cu) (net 42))
 (segment (start 167.012 103.075) (end 167.8792 103.9422) (width 0.25) (layer B.Cu) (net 42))
 (segment (start 158.5852 119.6042) (end 158.5852 120.820772) (width 0.25) (layer F.Cu) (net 44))
 (segment (start 158.5852 120.820772) (end 161.249999 123.485571) (width 0.25) (layer F.Cu) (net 44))
 (segment (start 158.9828 116.6) (end 158.9828 119.2066) (width 0.25) (layer B.Cu) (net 44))
 (segment (start 156.775 104.375) (end 158.9828 106.5828) (width 0.25) (layer B.Cu) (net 44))
 (segment (start 158.9828 106.5828) (end 158.9828 116.6) (width 0.25) (layer B.Cu) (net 44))
 (segment (start 154.2 104.375) (end 156.775 104.375) (width 0.25) (layer B.Cu) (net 44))
 (segment (start 158.9828 119.2066) (end 158.5852 119.6042) (width 0.25) (layer B.Cu) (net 44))
 (segment (start 165.621 112.7716) (end 167.007172 112.7716) (width 0.25) (layer F.Cu) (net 43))
 (segment (start 167.007172 112.7716) (end 169.485571 115.249999) (width 0.25) (layer F.Cu) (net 43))
 (segment (start 164.8186 111.456) (end 164.8186 111.9692) (width 0.25) (layer B.Cu) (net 43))
 (segment (start 157.0876 103.725) (end 164.8186 111.456) (width 0.25) (layer B.Cu) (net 43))
 (segment (start 154.2 103.725) (end 157.0876 103.725) (width 0.25) (layer B.Cu) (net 43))
 (segment (start 164.8186 111.9692) (end 165.621 112.7716) (width 0.25) (layer B.Cu) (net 43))
 (segment (start 167.404772 112.556) (end 169.883171 115.034399) (width 0.25) (layer F.Cu) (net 43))
 (segment (start 147 107.625) (end 145.668 107.625) (width 0.25) (layer B.Cu) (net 30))
 (segment (start 144.915 108.378) (end 144.0476 108.378) (width 0.25) (layer B.Cu) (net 30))
 (segment (start 145.668 107.625) (end 144.915 108.378) (width 0.25) (layer B.Cu) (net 30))
 (segment (start 147 100.475) (end 144.98 100.475) (width 0.25) (layer B.Cu) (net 38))
 (segment (start 143.311 93.218) (end 144.755 93.218) (width 0.25) (layer B.Cu) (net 38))
 (segment (start 142.676 93.853) (end 143.311 93.218) (width 0.25) (layer B.Cu) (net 38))
 (segment (start 142.676 98.171) (end 142.676 93.853) (width 0.25) (layer B.Cu) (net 38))
 (segment (start 144.98 100.475) (end 142.676 98.171) (width 0.25) (layer B.Cu) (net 38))
 (segment (start 151.867 94.154) (end 151.867 95.758) (width 0.25) (layer B.Cu) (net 4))
 (segment (start 148.979 95.758) (end 148.979 93.773) (width 0.25) (layer B.Cu) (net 4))
 (segment (start 148.424 93.218) (end 147.455 93.218) (width 0.25) (layer B.Cu) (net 4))
 (segment (start 148.979 93.773) (end 148.424 93.218) (width 0.25) (layer B.Cu) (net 4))
 (segment (start 148.979 95.758) (end 151.867 95.758) (width 0.25) (layer B.Cu) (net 4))
 (segment (start 154.2 102.425) (end 152.899 102.425) (width 0.25) (layer B.Cu) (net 4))
 (segment (start 151.867 101.393) (end 151.867 95.758) (width 0.25) (layer B.Cu) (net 4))
 (segment (start 152.899 102.425) (end 151.867 101.393) (width 0.25) (layer B.Cu) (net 4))
 (segment (start 144.0476 111.078) (end 148.311 111.078) (width 0.25) (layer B.Cu) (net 4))
 (segment (start 152.9 102.425) (end 154.2 102.425) (width 0.25) (layer B.Cu) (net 4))
 (segment (start 152.074 103.251) (end 152.9 102.425) (width 0.25) (layer B.Cu) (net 4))
 (segment (start 152.074 107.315) (end 152.074 103.251) (width 0.25) (layer B.Cu) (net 4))
 (segment (start 148.311 111.078) (end 152.074 107.315) (width 0.25) (layer B.Cu) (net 4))
 (segment (start 148.772 91.059) (end 151.867 94.154) (width 0.25) (layer B.Cu) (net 4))
 (segment (start 147.455 91.059) (end 148.772 91.059) (width 0.25) (layer B.Cu) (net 50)))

